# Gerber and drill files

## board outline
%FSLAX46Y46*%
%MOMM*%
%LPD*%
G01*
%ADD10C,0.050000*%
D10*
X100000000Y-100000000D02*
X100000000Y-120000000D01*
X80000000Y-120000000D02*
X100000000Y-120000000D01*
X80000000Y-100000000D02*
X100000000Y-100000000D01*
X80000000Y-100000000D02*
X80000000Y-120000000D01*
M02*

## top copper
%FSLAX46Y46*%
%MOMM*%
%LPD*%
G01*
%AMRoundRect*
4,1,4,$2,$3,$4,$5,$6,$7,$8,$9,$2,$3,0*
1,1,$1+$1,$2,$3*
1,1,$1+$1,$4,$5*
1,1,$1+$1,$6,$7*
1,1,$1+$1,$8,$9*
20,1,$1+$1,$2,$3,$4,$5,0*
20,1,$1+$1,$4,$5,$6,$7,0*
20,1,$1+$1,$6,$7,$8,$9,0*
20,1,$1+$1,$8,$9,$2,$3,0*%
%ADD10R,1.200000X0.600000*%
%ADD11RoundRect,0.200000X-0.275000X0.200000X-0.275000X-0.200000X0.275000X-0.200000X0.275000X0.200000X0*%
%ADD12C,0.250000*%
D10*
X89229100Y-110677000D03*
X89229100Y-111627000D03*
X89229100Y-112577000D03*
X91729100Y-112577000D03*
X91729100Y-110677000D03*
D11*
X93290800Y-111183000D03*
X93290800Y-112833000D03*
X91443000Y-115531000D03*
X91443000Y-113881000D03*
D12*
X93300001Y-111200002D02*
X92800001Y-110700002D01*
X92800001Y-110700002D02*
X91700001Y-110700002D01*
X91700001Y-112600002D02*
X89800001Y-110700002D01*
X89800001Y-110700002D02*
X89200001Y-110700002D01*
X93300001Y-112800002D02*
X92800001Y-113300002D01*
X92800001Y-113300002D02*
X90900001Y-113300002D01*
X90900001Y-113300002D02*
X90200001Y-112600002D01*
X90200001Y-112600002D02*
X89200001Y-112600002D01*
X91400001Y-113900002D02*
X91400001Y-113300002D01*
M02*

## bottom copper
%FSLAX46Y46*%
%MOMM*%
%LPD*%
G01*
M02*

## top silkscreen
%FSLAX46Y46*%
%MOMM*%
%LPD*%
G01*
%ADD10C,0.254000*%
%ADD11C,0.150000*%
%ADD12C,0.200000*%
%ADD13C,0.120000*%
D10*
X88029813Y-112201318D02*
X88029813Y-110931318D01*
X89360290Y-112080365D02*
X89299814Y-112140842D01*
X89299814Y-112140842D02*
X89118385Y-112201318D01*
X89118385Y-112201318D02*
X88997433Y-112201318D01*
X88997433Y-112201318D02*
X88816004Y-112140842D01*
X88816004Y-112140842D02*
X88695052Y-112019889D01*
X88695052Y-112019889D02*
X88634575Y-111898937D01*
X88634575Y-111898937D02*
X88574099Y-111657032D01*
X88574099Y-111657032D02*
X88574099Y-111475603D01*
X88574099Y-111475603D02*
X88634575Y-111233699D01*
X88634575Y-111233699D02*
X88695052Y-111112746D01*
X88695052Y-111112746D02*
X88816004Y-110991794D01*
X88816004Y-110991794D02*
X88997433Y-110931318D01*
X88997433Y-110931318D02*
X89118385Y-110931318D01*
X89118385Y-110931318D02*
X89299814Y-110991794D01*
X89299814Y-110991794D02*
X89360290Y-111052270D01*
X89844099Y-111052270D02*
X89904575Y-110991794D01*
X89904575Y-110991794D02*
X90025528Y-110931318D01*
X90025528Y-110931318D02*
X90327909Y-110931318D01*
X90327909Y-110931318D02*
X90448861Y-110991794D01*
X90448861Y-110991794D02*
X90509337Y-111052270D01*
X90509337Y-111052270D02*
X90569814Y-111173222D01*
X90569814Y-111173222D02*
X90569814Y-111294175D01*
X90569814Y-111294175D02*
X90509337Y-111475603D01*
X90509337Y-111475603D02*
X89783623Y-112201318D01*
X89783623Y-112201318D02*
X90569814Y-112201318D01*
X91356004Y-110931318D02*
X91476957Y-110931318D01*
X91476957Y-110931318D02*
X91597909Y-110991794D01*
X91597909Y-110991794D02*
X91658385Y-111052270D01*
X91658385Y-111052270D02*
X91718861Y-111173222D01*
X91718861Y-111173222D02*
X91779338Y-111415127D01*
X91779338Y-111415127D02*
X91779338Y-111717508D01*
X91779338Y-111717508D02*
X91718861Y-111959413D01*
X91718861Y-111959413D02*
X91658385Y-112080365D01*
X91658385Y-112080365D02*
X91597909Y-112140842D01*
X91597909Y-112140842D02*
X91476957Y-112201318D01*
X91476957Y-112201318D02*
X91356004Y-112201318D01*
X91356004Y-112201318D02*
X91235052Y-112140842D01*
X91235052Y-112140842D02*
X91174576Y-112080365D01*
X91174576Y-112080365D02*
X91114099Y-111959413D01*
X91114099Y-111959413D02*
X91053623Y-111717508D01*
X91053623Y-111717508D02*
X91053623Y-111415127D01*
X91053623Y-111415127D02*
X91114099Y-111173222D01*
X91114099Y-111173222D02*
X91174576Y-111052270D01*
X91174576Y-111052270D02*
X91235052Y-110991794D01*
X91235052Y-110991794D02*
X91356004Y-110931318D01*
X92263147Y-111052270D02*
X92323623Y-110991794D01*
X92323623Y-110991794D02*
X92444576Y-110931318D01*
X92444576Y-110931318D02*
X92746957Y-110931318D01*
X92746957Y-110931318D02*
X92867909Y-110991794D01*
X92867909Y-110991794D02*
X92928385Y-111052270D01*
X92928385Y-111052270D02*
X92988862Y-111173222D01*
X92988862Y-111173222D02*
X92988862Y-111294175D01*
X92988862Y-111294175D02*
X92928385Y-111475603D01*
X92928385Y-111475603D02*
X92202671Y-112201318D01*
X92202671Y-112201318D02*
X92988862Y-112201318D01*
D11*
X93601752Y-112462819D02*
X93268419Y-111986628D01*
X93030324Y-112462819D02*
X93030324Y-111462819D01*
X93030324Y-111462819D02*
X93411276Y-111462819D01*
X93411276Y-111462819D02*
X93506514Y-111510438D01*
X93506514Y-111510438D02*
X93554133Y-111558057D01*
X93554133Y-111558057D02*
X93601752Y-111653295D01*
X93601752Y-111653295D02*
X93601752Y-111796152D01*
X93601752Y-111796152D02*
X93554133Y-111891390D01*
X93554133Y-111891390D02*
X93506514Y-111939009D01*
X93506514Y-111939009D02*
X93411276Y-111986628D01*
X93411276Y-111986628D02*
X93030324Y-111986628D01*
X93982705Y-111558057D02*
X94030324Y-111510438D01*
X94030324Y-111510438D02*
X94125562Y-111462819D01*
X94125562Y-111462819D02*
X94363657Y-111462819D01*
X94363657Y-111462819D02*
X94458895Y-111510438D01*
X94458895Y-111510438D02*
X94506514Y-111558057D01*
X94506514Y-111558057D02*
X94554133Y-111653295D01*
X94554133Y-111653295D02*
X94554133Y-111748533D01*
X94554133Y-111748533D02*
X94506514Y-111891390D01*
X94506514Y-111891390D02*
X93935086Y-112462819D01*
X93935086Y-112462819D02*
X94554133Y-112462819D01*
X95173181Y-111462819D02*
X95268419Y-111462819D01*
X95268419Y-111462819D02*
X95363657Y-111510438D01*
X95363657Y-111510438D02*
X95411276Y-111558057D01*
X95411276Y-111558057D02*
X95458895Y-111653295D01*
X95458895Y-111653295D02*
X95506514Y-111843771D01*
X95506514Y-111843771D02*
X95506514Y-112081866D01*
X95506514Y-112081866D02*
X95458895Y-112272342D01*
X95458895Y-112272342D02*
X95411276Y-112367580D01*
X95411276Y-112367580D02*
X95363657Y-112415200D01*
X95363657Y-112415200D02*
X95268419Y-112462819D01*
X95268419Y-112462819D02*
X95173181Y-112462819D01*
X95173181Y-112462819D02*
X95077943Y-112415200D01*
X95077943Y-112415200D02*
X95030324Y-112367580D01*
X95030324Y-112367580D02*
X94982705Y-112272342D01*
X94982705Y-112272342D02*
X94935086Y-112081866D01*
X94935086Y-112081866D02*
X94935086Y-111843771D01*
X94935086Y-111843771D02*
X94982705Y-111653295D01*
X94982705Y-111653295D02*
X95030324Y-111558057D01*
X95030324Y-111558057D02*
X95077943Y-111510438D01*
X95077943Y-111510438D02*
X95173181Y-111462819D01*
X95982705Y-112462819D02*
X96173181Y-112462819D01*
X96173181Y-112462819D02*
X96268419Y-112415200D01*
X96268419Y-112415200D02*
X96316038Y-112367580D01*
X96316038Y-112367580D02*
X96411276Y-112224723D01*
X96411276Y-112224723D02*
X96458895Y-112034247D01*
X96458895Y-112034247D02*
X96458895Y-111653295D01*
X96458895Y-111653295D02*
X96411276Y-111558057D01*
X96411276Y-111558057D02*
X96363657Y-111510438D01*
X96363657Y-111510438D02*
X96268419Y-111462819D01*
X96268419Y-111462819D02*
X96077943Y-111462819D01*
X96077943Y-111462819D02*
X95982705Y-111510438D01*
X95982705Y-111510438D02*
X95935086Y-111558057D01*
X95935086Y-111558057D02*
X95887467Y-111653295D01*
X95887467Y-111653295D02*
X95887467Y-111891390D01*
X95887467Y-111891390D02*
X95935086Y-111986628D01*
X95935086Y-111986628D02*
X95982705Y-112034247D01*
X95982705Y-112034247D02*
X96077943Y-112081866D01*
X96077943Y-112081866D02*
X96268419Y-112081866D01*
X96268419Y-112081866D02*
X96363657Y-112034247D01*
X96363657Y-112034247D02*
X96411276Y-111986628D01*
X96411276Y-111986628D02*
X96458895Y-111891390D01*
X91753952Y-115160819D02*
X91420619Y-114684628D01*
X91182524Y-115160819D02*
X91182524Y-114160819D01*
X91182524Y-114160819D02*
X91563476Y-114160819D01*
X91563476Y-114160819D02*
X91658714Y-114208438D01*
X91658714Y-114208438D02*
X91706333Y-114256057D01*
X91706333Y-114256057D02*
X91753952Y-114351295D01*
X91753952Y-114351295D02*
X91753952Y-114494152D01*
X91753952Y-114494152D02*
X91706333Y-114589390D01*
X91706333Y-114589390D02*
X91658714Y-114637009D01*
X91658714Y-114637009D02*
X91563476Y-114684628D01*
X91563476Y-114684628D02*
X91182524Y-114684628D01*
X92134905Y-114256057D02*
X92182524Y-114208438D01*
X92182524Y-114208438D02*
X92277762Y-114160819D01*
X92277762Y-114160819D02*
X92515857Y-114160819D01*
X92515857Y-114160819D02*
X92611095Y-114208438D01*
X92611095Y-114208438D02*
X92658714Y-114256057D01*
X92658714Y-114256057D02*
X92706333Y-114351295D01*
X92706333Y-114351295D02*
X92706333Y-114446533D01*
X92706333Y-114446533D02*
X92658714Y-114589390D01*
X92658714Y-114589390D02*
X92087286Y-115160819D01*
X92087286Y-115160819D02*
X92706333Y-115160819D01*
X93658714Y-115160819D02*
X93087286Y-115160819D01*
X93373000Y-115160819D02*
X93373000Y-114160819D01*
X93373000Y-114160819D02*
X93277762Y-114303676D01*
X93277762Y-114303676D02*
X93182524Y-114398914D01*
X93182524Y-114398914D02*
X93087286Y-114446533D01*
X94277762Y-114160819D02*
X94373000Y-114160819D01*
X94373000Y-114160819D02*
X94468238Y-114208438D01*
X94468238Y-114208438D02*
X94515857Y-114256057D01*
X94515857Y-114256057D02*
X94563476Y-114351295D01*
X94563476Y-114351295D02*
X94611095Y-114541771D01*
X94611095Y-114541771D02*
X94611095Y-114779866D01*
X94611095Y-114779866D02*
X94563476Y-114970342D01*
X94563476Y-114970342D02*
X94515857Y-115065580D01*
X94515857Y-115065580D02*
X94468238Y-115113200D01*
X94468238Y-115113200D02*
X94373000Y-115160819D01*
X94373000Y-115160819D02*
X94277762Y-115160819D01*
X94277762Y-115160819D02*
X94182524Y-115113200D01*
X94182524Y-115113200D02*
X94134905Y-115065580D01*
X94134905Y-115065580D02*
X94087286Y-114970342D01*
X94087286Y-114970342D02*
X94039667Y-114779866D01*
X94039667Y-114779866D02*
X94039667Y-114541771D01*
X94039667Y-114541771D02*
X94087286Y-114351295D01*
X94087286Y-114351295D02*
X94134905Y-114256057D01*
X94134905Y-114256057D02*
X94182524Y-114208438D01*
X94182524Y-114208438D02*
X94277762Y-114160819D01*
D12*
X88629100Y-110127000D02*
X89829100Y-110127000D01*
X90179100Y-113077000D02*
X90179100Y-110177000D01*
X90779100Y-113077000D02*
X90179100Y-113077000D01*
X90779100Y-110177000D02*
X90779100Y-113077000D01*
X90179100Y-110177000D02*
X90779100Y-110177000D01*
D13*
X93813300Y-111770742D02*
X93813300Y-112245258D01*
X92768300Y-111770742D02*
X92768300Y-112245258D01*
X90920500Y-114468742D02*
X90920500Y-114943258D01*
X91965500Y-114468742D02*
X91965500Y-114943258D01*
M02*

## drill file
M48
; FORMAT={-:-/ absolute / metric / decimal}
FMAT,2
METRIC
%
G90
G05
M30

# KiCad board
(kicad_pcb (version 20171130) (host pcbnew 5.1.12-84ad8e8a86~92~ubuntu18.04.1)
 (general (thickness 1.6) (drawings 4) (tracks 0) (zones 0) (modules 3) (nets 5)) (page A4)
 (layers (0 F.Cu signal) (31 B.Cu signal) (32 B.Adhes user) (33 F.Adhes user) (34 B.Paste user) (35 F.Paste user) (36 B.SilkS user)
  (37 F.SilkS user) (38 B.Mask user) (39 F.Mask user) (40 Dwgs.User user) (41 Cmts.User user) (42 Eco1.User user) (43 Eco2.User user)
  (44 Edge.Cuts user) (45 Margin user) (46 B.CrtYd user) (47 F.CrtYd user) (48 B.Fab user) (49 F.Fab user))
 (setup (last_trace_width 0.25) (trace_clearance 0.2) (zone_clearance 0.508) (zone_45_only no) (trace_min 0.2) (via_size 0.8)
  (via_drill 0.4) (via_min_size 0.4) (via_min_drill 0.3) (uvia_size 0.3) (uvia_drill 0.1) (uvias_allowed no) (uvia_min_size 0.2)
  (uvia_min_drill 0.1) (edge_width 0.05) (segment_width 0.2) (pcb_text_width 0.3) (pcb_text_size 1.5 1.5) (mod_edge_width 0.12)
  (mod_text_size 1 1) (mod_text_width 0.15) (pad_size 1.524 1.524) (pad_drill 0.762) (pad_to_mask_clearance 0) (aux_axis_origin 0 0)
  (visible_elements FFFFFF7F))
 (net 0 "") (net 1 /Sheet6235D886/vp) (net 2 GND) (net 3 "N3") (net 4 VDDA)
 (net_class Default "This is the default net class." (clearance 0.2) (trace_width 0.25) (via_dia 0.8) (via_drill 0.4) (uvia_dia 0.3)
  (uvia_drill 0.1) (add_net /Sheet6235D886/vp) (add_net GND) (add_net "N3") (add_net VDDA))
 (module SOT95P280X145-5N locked (layer F.Cu) (at 90.479100 111.627000)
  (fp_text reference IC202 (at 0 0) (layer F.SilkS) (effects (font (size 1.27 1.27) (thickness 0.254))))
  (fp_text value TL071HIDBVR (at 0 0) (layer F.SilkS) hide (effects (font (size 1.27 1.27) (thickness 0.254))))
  (fp_line (start -1.85 -1.5) (end -0.65 -1.5) (layer F.SilkS) (width 0.2))
  (fp_line (start -0.3 1.45) (end -0.3 -1.45) (layer F.SilkS) (width 0.2))
  (fp_line (start 0.3 1.45) (end -0.3 1.45) (layer F.SilkS) (width 0.2))
  (fp_line (start 0.3 -1.45) (end 0.3 1.45) (layer F.SilkS) (width 0.2))
  (fp_line (start -0.3 -1.45) (end 0.3 -1.45) (layer F.SilkS) (width 0.2))
  (pad 1 smd rect (at -1.25 -0.95 90.000000) (size 0.6 1.2) (layers F.Cu F.Mask F.Paste) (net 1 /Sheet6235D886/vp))
  (pad 2 smd rect (at -1.25 0 90.000000) (size 0.6 1.2) (layers F.Cu F.Mask F.Paste) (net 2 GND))
  (pad 3 smd rect (at -1.25 0.95 90.000000) (size 0.6 1.2) (layers F.Cu F.Mask F.Paste) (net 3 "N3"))
  (pad 4 smd rect (at 1.25 0.95 90.000000) (size 0.6 1.2) (layers F.Cu F.Mask F.Paste) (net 1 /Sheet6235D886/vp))
  (pad 5 smd rect (at 1.25 -0.95 90.000000) (size 0.6 1.2) (layers F.Cu F.Mask F.Paste) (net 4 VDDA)))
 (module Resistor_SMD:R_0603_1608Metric (layer F.Cu) (at 93.290800 112.008000 270.000000)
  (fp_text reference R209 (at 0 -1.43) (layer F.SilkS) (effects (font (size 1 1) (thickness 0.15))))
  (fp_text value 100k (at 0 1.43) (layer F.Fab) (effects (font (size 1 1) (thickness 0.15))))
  (fp_line (start -0.237258 -0.5225) (end 0.237258 -0.5225) (layer F.SilkS) (width 0.12))
  (fp_line (start -0.237258 0.5225) (end 0.237258 0.5225) (layer F.SilkS) (width 0.12))
  (pad 1 smd roundrect (at -0.825 0 270.000000) (size 0.8 0.95) (layers F.Cu F.Mask F.Paste) (roundrect_rratio 0.25) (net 4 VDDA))
  (pad 2 smd roundrect (at 0.825 0 270.000000) (size 0.8 0.95) (layers F.Cu F.Mask F.Paste) (roundrect_rratio 0.25) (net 3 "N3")))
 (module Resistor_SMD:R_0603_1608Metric (layer F.Cu) (at 91.443000 114.706000 270.000000)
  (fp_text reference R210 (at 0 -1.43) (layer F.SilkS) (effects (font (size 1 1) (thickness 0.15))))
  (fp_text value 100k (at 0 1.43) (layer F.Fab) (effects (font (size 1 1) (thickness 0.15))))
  (fp_line (start -0.237258 0.5225) (end 0.237258 0.5225) (layer F.SilkS) (width 0.12))
  (fp_line (start -0.237258 -0.5225) (end 0.237258 -0.5225) (layer F.SilkS) (width 0.12))
  (pad 2 smd roundrect (at 0.825 0 270.000000) (size 0.8 0.95) (layers F.Cu F.Mask F.Paste) (roundrect_rratio 0.25) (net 2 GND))
  (pad 1 smd roundrect (at -0.825 0 270.000000) (size 0.8 0.95) (layers F.Cu F.Mask F.Paste) (roundrect_rratio 0.25) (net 3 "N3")))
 (gr_line (start 100 100) (end 100 120) (layer Edge.Cuts) (width 0.05))
 (gr_line (start 80 120) (end 100 120) (layer Edge.Cuts) (width 0.05))
 (gr_line (start 80 100) (end 100 100) (layer Edge.Cuts) (width 0.05))
 (gr_line (start 80 100) (end 80 120) (layer Edge.Cuts) (width 0.05))
 (segment (start 93.300001 111.200002) (end 92.800001 110.700002) (width 0.250000) (layer F.Cu) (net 4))
 (segment (start 92.800001 110.700002) (end 91.700001 110.700002) (width 0.250000) (layer F.Cu) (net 4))
 (segment (start 91.700001 112.600002) (end 89.800001 110.700002) (width 0.250000) (layer F.Cu) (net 1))
 (segment (start 89.800001 110.700002) (end 89.200001 110.700002) (width 0.250000) (layer F.Cu) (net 1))
 (segment (start 93.300001 112.800002) (end 92.800001 113.300002) (width 0.250000) (layer F.Cu) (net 3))
 (segment (start 92.800001 113.300002) (end 90.900001 113.300002) (width 0.250000) (layer F.Cu) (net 3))
 (segment (start 90.900001 113.300002) (end 90.200001 112.600002) (width 0.250000) (layer F.Cu) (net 3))
 (segment (start 90.200001 112.600002) (end 89.200001 112.600002) (width 0.250000) (layer F.Cu) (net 3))
 (segment (start 91.400001 113.900002) (end 91.400001 113.300002) (width 0.250000) (layer F.Cu) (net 3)))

